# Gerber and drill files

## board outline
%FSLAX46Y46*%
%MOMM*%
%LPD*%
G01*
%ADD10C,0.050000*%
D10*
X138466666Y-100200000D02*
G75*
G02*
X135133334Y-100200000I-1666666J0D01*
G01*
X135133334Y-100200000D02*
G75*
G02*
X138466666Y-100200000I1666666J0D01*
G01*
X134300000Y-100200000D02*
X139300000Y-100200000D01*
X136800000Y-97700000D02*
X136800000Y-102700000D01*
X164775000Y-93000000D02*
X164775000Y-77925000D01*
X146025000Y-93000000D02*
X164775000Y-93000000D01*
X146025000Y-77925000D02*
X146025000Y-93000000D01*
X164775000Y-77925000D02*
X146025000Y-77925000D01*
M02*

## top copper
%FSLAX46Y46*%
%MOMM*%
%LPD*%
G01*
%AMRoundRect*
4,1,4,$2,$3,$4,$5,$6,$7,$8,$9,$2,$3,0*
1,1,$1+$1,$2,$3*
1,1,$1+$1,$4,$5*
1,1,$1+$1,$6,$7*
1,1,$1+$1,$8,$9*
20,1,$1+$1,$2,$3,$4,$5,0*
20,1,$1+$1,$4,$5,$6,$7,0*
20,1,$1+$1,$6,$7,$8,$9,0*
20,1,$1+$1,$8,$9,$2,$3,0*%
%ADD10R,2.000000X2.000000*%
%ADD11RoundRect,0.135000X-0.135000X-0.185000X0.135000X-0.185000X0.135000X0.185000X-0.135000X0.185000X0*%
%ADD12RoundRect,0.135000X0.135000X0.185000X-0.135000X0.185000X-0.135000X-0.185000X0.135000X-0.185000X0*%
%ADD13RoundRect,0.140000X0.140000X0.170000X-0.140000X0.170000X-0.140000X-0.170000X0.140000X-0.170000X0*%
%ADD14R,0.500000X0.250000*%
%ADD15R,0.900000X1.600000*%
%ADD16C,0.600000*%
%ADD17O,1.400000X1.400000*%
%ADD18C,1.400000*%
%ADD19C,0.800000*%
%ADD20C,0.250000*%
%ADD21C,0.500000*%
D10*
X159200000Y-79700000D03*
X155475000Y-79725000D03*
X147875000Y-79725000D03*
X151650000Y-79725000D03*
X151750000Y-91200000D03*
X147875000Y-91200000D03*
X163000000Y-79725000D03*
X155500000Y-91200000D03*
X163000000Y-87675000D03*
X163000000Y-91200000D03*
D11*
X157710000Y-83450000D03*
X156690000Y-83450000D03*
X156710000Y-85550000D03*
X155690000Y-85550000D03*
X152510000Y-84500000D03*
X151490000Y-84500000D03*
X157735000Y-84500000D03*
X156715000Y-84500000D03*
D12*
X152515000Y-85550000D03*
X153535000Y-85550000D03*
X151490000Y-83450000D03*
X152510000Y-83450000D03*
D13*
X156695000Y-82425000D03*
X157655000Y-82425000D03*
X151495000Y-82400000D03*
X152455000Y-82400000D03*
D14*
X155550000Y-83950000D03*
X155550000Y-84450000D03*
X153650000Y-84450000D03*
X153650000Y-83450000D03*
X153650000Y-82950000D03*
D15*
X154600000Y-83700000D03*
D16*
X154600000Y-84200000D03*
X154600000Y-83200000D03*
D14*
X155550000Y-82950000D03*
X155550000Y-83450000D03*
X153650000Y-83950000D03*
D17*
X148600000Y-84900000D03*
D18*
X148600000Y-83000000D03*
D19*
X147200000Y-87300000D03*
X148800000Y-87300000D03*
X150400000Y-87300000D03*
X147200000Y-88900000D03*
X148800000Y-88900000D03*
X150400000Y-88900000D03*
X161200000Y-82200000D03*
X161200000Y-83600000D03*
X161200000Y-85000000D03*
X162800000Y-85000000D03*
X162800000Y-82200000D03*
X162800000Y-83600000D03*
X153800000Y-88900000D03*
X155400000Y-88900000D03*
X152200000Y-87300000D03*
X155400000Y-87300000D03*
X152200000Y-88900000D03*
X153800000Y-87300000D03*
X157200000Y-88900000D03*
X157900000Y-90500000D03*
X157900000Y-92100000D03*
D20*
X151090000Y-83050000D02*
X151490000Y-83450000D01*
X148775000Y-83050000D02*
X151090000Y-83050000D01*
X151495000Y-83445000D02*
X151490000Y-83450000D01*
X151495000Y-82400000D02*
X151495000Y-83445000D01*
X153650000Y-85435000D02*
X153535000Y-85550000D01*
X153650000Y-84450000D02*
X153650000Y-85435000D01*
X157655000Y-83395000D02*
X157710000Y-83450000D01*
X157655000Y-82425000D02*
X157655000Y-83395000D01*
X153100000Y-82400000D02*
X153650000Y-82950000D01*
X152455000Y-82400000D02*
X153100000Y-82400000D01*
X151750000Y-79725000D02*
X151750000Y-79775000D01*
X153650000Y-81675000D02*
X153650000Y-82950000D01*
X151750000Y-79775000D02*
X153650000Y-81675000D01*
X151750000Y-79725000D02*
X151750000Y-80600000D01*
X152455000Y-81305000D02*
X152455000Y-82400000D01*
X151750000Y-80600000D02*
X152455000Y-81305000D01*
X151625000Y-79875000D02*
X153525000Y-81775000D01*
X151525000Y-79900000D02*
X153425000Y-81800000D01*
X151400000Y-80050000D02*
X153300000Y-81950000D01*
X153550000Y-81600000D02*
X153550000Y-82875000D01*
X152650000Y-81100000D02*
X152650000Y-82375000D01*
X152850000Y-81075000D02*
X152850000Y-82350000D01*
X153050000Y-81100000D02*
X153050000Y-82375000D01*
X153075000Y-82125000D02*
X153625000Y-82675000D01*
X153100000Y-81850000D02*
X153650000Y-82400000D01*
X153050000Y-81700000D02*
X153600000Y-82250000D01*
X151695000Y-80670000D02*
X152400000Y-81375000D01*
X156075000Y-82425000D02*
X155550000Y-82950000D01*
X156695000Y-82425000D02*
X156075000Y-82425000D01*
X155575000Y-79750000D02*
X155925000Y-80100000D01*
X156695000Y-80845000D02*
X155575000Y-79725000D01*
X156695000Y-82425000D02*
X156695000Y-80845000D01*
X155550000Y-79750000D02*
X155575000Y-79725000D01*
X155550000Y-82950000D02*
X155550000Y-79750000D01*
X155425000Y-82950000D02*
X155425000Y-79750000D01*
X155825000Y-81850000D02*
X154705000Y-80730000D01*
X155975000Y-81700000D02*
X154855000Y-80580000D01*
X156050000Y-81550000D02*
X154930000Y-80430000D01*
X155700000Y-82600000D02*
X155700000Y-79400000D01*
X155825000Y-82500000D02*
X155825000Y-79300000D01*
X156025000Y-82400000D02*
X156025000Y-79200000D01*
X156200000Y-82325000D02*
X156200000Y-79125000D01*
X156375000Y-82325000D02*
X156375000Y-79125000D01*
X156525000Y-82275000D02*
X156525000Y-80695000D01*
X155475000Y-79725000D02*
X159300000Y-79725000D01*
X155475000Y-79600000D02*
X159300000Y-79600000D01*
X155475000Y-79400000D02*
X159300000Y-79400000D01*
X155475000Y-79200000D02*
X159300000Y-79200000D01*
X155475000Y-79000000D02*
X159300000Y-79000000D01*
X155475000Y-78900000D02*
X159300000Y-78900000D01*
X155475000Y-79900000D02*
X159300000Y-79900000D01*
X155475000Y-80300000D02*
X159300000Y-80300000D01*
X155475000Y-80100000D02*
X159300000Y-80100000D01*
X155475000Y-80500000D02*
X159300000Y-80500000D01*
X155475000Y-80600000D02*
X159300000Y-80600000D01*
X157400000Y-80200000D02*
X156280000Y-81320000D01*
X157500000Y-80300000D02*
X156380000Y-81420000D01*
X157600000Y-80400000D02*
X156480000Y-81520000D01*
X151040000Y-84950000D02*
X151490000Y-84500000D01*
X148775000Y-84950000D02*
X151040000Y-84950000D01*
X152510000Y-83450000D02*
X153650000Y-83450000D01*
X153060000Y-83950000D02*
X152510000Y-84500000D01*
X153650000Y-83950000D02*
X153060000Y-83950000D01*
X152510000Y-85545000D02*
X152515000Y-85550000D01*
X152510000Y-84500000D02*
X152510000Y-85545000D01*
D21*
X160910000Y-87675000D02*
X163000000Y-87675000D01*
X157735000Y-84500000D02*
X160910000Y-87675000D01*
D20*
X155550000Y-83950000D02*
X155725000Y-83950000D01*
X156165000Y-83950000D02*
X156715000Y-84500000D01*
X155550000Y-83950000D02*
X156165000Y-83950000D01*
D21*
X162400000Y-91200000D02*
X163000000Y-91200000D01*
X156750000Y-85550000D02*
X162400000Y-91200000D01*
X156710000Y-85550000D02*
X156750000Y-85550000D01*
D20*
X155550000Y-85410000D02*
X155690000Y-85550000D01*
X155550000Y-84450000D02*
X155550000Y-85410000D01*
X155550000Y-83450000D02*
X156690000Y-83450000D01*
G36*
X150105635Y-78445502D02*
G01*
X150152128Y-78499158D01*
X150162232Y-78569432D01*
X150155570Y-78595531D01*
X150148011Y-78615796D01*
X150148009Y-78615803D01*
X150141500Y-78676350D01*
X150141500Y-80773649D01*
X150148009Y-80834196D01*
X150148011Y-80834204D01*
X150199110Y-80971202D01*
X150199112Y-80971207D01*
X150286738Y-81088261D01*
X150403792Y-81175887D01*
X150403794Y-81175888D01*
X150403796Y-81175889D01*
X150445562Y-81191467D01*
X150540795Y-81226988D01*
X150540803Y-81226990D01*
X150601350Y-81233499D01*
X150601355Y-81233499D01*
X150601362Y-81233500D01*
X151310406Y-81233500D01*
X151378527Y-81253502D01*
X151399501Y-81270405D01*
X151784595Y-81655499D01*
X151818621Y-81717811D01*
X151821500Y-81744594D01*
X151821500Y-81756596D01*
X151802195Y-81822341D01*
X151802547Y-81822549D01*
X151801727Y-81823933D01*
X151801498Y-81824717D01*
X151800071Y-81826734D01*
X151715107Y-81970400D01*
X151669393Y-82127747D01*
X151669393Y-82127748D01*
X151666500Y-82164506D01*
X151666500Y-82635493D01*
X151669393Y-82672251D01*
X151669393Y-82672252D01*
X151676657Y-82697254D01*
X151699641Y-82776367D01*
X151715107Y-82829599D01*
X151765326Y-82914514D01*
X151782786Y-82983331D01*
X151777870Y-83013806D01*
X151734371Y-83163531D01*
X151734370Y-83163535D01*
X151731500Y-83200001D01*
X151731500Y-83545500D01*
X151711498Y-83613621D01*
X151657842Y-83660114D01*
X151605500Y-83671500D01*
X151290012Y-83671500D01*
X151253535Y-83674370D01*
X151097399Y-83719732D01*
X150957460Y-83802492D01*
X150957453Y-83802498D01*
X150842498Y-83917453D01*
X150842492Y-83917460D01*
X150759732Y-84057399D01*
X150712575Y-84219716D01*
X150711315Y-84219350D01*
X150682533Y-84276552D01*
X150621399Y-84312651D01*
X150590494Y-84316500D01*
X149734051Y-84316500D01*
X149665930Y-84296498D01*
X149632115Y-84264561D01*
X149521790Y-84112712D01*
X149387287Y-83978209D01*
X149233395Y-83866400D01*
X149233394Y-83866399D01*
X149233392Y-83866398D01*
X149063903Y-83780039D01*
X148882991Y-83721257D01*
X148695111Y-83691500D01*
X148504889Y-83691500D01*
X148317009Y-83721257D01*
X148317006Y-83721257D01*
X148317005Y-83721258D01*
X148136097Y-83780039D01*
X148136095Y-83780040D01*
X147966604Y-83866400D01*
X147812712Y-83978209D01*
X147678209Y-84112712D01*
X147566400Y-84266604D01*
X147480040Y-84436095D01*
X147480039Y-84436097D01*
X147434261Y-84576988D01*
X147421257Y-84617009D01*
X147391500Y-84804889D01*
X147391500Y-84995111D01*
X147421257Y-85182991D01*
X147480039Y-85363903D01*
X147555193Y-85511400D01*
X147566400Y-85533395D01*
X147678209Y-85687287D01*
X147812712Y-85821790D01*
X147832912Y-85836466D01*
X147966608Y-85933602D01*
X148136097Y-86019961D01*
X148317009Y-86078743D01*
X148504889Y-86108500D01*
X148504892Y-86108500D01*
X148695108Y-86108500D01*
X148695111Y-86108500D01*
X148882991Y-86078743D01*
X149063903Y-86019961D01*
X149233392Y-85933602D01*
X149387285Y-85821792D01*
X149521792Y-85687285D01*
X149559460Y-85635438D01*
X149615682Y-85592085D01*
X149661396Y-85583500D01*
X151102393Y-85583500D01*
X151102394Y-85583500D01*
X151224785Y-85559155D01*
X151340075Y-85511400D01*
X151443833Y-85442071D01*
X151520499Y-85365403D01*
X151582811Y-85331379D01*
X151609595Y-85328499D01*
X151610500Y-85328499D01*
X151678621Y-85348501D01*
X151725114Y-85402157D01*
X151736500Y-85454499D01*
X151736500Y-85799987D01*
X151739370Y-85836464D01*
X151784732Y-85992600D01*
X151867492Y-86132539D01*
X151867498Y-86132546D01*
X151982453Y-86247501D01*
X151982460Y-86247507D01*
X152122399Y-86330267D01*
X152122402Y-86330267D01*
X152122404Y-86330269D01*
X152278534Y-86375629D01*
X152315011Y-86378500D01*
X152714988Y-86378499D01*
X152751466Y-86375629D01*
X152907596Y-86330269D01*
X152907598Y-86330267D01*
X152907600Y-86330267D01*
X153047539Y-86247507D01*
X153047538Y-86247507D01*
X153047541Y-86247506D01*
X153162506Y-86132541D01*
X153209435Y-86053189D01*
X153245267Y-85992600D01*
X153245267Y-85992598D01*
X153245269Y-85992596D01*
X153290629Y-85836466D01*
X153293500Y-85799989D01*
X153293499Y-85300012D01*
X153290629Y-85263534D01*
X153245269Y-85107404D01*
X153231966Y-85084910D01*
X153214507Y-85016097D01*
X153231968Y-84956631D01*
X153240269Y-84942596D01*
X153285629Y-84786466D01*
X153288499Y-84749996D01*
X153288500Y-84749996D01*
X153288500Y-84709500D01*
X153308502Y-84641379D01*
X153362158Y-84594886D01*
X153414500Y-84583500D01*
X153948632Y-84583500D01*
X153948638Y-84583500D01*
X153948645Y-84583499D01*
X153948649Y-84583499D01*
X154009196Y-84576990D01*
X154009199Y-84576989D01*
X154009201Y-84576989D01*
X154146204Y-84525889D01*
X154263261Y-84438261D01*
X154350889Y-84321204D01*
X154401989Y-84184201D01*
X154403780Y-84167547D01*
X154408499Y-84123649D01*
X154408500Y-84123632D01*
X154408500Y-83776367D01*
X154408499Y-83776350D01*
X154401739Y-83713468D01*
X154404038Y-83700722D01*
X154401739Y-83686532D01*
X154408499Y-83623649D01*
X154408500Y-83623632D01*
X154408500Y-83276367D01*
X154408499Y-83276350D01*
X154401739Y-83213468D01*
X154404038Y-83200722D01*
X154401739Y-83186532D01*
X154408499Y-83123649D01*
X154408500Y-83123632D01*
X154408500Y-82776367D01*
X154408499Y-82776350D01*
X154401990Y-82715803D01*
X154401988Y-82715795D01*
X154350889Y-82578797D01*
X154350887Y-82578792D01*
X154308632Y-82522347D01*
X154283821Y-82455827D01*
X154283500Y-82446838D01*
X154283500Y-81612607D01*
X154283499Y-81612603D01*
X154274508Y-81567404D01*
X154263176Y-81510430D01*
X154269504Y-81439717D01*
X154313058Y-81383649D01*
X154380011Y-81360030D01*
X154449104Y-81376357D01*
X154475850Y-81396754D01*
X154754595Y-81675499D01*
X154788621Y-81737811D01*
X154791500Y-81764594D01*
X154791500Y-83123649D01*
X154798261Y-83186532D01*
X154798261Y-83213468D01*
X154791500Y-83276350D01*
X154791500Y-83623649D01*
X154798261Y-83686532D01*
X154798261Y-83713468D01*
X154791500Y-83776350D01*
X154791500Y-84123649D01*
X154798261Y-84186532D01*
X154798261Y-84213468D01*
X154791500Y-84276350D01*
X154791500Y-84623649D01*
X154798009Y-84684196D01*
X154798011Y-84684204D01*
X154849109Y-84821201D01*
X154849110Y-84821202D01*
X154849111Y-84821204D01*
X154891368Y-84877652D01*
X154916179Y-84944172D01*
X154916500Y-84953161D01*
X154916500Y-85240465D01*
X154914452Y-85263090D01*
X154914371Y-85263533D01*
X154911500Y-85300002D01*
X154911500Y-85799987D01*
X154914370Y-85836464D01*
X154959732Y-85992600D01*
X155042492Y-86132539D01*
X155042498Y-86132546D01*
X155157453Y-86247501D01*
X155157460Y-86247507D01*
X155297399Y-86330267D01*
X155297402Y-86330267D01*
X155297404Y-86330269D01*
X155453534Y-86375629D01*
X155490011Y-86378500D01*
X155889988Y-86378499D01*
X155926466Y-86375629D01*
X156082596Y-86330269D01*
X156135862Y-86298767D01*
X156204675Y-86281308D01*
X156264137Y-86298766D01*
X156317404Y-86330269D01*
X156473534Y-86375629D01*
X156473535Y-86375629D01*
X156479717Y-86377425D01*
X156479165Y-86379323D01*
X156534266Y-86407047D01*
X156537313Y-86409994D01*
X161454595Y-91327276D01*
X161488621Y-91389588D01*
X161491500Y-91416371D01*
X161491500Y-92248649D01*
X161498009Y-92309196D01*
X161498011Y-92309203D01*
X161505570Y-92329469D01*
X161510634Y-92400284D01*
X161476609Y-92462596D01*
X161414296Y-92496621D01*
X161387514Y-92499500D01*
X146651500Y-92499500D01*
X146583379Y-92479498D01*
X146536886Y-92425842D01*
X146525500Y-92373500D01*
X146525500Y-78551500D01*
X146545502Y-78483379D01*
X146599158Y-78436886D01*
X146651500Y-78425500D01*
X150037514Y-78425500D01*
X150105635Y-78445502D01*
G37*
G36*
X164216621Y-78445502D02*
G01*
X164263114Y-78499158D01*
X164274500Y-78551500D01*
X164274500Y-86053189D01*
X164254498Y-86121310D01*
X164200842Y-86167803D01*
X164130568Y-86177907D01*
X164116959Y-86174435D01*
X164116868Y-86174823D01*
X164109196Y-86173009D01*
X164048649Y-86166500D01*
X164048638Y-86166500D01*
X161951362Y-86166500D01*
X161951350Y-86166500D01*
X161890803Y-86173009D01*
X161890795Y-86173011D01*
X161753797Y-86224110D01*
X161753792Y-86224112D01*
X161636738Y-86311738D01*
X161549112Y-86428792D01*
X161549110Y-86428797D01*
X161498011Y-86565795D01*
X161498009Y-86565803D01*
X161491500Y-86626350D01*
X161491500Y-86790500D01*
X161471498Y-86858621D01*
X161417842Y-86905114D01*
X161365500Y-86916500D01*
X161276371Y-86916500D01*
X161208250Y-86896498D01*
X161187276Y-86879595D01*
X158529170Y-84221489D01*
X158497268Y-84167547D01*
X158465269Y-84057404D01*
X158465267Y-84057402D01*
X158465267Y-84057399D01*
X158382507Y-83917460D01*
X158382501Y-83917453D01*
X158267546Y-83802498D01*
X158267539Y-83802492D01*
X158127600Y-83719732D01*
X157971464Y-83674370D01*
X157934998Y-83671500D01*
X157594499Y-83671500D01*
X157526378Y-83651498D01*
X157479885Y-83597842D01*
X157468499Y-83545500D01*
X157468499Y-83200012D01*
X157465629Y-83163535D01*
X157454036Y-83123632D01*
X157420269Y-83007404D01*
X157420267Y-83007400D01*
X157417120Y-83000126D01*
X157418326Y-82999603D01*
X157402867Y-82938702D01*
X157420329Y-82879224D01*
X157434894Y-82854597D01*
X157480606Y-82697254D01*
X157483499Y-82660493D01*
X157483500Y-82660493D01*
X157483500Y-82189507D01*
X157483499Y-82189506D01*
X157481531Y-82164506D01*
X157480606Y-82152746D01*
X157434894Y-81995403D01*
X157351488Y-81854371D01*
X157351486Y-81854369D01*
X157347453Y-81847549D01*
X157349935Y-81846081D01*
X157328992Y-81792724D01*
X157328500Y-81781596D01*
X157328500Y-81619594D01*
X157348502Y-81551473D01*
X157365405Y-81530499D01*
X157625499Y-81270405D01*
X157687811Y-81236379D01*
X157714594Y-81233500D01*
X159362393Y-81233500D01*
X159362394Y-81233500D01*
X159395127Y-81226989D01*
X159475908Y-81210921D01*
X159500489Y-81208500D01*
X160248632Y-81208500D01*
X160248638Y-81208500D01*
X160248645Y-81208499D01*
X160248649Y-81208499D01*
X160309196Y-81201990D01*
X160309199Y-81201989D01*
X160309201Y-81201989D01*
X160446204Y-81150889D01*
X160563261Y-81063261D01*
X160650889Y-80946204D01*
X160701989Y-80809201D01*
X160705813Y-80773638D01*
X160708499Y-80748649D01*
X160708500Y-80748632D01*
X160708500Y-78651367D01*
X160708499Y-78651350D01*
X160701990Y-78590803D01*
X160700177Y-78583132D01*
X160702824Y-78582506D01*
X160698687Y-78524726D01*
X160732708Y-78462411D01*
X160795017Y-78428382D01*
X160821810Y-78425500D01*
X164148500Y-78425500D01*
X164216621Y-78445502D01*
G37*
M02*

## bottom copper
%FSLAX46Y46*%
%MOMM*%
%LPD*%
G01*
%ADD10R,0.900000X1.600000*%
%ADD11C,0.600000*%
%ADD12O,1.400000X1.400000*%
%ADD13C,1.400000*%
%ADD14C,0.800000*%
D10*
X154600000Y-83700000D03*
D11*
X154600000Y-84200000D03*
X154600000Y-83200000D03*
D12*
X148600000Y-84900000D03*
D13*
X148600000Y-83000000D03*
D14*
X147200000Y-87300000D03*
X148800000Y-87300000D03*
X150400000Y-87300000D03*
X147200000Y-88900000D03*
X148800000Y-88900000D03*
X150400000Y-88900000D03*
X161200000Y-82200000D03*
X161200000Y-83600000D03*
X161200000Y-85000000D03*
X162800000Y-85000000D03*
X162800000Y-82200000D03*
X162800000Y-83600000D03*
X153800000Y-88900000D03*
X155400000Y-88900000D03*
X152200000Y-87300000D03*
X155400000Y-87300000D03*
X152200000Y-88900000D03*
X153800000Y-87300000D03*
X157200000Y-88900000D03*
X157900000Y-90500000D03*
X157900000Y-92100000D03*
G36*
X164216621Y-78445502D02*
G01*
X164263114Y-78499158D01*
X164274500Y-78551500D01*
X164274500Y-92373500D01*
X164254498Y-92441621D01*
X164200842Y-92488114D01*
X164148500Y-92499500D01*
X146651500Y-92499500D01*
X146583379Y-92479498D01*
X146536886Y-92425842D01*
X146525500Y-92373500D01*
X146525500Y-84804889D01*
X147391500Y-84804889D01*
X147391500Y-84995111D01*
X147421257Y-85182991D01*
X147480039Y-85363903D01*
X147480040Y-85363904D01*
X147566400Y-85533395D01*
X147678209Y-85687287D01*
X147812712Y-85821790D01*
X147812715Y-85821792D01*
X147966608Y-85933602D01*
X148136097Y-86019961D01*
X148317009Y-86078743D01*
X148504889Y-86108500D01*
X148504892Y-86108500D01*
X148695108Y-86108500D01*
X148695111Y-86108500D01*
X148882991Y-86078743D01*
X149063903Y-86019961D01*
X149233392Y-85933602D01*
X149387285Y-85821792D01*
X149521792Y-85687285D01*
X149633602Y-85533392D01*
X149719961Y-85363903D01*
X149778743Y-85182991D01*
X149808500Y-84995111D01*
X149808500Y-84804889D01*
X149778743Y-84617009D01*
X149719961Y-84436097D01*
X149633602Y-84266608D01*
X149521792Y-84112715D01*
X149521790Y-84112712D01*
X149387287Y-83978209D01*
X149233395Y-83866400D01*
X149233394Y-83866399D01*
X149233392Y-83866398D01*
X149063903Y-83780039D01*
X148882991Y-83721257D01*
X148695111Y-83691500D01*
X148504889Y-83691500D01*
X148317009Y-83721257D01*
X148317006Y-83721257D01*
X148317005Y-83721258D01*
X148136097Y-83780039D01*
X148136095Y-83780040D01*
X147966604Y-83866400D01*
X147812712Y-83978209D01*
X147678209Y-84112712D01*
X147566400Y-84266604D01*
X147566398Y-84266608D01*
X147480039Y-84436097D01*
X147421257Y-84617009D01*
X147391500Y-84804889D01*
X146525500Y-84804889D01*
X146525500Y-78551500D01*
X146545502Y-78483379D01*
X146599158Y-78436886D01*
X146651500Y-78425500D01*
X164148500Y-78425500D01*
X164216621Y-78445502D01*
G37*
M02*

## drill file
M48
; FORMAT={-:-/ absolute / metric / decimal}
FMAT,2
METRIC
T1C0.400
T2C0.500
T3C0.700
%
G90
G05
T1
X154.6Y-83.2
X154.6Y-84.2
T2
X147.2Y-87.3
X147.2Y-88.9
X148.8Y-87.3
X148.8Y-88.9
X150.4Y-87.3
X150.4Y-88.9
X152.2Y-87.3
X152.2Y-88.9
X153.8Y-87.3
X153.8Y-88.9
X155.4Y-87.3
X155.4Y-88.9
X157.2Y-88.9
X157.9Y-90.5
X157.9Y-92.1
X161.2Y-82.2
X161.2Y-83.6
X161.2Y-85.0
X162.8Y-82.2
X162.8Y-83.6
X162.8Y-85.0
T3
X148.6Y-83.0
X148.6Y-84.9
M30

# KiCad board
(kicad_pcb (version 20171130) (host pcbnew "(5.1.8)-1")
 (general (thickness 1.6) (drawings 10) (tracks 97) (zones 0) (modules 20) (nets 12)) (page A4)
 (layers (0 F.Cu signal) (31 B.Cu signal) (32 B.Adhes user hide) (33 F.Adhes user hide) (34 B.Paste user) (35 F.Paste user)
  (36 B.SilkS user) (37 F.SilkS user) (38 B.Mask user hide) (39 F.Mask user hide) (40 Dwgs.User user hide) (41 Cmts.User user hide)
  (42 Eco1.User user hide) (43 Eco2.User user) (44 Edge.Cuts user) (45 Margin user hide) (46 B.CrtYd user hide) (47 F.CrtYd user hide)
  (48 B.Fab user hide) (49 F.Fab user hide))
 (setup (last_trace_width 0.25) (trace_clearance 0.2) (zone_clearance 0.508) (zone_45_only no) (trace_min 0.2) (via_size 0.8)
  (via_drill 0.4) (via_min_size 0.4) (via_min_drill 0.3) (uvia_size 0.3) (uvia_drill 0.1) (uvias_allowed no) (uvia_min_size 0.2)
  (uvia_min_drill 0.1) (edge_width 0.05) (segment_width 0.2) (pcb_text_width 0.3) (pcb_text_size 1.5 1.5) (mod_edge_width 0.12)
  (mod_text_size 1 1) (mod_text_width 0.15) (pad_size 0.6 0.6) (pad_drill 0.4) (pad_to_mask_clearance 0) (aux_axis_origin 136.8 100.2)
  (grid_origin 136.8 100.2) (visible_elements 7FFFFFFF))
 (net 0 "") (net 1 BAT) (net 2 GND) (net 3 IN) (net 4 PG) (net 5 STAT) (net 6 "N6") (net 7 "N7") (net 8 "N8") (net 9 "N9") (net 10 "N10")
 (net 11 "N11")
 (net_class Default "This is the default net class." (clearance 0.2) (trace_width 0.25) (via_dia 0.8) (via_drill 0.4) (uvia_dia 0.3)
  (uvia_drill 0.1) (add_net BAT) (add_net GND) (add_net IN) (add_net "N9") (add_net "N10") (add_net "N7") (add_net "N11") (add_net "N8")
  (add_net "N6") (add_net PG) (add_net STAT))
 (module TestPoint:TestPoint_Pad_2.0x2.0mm (layer F.Cu) (at 159.2 79.7)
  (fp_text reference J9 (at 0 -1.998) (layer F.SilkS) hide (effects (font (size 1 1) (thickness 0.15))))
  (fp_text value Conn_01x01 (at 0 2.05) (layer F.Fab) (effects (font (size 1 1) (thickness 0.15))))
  (pad 1 smd rect (at 0 0) (size 2 2) (layers F.Cu F.Mask) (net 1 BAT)))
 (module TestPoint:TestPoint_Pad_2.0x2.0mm (layer F.Cu) (at 155.475 79.725)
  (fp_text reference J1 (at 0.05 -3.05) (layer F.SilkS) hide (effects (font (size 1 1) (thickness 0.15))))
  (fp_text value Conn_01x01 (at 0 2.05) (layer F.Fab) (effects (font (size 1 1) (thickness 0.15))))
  (pad 1 smd rect (at 0 0) (size 2 2) (layers F.Cu F.Mask) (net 1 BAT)))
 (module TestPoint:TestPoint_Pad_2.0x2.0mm (layer F.Cu) (at 147.875 79.725)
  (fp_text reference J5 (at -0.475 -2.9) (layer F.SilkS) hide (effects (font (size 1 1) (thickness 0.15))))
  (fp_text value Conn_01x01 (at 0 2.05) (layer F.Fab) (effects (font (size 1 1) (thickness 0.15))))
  (pad 1 smd rect (at 0 0) (size 2 2) (layers F.Cu F.Mask) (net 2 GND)))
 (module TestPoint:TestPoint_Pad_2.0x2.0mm (layer F.Cu) (at 151.65 79.725)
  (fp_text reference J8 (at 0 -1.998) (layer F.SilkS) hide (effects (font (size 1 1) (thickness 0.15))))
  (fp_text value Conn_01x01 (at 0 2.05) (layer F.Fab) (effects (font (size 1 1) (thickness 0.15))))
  (pad 1 smd rect (at 0 0) (size 2 2) (layers F.Cu F.Mask) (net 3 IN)))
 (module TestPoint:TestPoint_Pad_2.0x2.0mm (layer F.Cu) (at 151.75 91.2)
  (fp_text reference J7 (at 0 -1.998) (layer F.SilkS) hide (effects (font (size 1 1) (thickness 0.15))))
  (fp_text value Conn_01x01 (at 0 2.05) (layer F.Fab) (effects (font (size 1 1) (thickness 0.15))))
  (pad 1 smd rect (at 0 0) (size 2 2) (layers F.Cu F.Mask) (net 2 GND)))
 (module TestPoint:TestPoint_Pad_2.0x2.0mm (layer F.Cu) (at 147.875 91.2)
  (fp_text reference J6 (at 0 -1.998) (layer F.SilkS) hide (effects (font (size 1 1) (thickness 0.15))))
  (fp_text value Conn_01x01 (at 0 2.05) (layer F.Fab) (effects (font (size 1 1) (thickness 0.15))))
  (pad 1 smd rect (at 0 0) (size 2 2) (layers F.Cu F.Mask) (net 2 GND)))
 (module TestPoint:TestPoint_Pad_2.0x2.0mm (layer F.Cu) (at 163 79.725)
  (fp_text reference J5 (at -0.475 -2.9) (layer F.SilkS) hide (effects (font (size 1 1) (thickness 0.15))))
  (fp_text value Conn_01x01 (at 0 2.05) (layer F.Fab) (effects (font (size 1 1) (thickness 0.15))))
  (pad 1 smd rect (at 0 0) (size 2 2) (layers F.Cu F.Mask) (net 2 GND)))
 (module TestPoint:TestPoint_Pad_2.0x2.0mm (layer F.Cu) (at 155.5 91.2)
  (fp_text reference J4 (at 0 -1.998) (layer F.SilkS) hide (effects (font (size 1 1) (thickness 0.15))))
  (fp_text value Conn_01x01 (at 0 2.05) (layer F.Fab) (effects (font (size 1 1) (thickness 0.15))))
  (pad 1 smd rect (at 0 0) (size 2 2) (layers F.Cu F.Mask) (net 2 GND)))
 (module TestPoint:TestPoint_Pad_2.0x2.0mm (layer F.Cu) (at 163 87.675)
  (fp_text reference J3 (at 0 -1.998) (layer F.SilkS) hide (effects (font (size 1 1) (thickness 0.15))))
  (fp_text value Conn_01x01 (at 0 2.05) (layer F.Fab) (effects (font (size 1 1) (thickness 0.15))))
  (pad 1 smd rect (at 0 0) (size 2 2) (layers F.Cu F.Mask) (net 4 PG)))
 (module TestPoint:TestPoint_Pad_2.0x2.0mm (layer F.Cu) (at 163 91.2)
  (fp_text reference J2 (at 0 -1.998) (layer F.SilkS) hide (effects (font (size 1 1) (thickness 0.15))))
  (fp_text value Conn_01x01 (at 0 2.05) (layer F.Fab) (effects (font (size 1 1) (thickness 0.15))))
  (pad 1 smd rect (at 0 0) (size 2 2) (layers F.Cu F.Mask) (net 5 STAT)))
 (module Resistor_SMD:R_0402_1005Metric (layer F.Cu) (at 157.2 83.45)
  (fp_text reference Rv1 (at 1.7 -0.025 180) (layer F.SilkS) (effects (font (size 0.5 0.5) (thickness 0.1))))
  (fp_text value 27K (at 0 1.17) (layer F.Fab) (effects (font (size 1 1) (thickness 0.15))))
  (pad 2 smd roundrect (at 0.51 0) (size 0.54 0.64) (layers F.Cu F.Paste F.Mask) (roundrect_rratio 0.25) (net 2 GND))
  (pad 1 smd roundrect (at -0.51 0) (size 0.54 0.64) (layers F.Cu F.Paste F.Mask) (roundrect_rratio 0.25) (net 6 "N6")))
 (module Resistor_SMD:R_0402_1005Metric (layer F.Cu) (at 156.2 85.55)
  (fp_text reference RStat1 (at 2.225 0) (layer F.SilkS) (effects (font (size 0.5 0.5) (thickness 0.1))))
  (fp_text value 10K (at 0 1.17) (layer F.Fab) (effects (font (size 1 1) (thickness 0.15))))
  (pad 2 smd roundrect (at 0.51 0) (size 0.54 0.64) (layers F.Cu F.Paste F.Mask) (roundrect_rratio 0.25) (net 5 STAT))
  (pad 1 smd roundrect (at -0.51 0) (size 0.54 0.64) (layers F.Cu F.Paste F.Mask) (roundrect_rratio 0.25) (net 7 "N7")))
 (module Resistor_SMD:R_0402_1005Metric (layer F.Cu) (at 152 84.5)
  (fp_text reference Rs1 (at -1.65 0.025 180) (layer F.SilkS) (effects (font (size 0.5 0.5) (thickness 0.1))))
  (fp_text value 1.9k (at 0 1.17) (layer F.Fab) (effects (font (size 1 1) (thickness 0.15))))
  (pad 2 smd roundrect (at 0.51 0) (size 0.54 0.64) (layers F.Cu F.Paste F.Mask) (roundrect_rratio 0.25) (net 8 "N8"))
  (pad 1 smd roundrect (at -0.51 0) (size 0.54 0.64) (layers F.Cu F.Paste F.Mask) (roundrect_rratio 0.25) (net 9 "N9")))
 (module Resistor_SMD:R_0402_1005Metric (layer F.Cu) (at 157.225 84.5)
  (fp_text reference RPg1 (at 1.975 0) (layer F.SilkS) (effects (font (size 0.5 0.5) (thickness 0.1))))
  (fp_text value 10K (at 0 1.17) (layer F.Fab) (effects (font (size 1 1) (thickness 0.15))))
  (pad 2 smd roundrect (at 0.51 0) (size 0.54 0.64) (layers F.Cu F.Paste F.Mask) (roundrect_rratio 0.25) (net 4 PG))
  (pad 1 smd roundrect (at -0.51 0) (size 0.54 0.64) (layers F.Cu F.Paste F.Mask) (roundrect_rratio 0.25) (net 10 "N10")))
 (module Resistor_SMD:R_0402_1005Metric (layer F.Cu) (at 153.025 85.55 180)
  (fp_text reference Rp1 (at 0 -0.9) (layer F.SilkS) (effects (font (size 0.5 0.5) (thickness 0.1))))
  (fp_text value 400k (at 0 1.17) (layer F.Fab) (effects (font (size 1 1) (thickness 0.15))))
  (pad 2 smd roundrect (at 0.51 0 180) (size 0.54 0.64) (layers F.Cu F.Paste F.Mask) (roundrect_rratio 0.25) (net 8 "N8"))
  (pad 1 smd roundrect (at -0.51 0 180) (size 0.54 0.64) (layers F.Cu F.Paste F.Mask) (roundrect_rratio 0.25) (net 2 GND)))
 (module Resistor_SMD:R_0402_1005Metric (layer F.Cu) (at 152 83.45 180)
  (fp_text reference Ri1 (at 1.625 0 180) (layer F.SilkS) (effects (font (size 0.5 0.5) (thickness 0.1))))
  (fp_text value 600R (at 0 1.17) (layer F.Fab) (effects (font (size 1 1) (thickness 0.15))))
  (pad 2 smd roundrect (at 0.51 0 180) (size 0.54 0.64) (layers F.Cu F.Paste F.Mask) (roundrect_rratio 0.25) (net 2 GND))
  (pad 1 smd roundrect (at -0.51 0 180) (size 0.54 0.64) (layers F.Cu F.Paste F.Mask) (roundrect_rratio 0.25) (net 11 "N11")))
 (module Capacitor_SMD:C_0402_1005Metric (layer F.Cu) (at 157.175 82.425 180)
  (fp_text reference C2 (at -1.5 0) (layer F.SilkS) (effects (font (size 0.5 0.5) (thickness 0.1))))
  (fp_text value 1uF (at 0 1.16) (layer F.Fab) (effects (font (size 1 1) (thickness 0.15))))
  (pad 2 smd roundrect (at 0.48 0 180) (size 0.56 0.62) (layers F.Cu F.Paste F.Mask) (roundrect_rratio 0.25) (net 1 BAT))
  (pad 1 smd roundrect (at -0.48 0 180) (size 0.56 0.62) (layers F.Cu F.Paste F.Mask) (roundrect_rratio 0.25) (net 2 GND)))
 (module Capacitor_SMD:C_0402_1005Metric (layer F.Cu) (at 151.975 82.4 180)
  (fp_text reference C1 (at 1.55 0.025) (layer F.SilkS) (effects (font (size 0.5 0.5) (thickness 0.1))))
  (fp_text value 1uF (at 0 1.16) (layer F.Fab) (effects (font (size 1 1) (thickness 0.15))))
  (pad 2 smd roundrect (at 0.48 0 180) (size 0.56 0.62) (layers F.Cu F.Paste F.Mask) (roundrect_rratio 0.25) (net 2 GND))
  (pad 1 smd roundrect (at -0.48 0 180) (size 0.56 0.62) (layers F.Cu F.Paste F.Mask) (roundrect_rratio 0.25) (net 3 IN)))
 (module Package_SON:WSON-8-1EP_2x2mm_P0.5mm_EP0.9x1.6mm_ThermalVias (layer F.Cu) (at 154.6 83.7)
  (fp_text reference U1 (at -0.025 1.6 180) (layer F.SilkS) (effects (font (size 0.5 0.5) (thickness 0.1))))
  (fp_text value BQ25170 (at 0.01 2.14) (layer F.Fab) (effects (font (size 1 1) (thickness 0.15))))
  (pad "" smd rect (at 0 -0.4) (size 0.75 0.65) (layers F.Paste))
  (pad "" smd rect (at 0 0.4) (size 0.75 0.65) (layers F.Paste))
  (pad 9 smd rect (at 0 0) (size 0.9 1.6) (layers B.Cu) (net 2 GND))
  (pad 6 smd rect (at 0.95 0.25) (size 0.5 0.25) (layers F.Cu F.Paste F.Mask) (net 10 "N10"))
  (pad 5 smd rect (at 0.95 0.75) (size 0.5 0.25) (layers F.Cu F.Paste F.Mask) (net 7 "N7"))
  (pad 4 smd rect (at -0.95 0.75) (size 0.5 0.25) (layers F.Cu F.Paste F.Mask) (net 2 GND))
  (pad 2 smd rect (at -0.95 -0.25) (size 0.5 0.25) (layers F.Cu F.Paste F.Mask) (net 11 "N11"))
  (pad 1 smd rect (at -0.95 -0.75) (size 0.5 0.25) (layers F.Cu F.Paste F.Mask) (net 3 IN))
  (pad 9 smd rect (at 0 0) (size 0.9 1.6) (layers F.Cu F.Mask) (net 2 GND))
  (pad 9 thru_hole circle (at 0 0.5) (size 0.6 0.6) (drill 0.4) (layers *.Cu) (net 2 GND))
  (pad 9 thru_hole circle (at 0 -0.5) (size 0.6 0.6) (drill 0.4) (layers *.Cu) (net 2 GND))
  (pad 8 smd rect (at 0.95 -0.75) (size 0.5 0.25) (layers F.Cu F.Paste F.Mask) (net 1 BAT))
  (pad 7 smd rect (at 0.95 -0.25) (size 0.5 0.25) (layers F.Cu F.Paste F.Mask) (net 6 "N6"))
  (pad 3 smd rect (at -0.95 0.25) (size 0.5 0.25) (layers F.Cu F.Paste F.Mask) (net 8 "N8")))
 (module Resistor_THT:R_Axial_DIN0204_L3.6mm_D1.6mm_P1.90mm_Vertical (layer F.Cu) (at 148.6 83 270)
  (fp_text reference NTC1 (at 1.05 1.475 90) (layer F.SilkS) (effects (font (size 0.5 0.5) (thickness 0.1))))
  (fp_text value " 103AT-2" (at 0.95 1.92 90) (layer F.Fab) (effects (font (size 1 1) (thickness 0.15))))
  (pad 2 thru_hole oval (at 1.9 0 270) (size 1.4 1.4) (drill 0.7) (layers *.Cu *.Mask) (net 9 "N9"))
  (pad 1 thru_hole circle (at 0 0 270) (size 1.4 1.4) (drill 0.7) (layers *.Cu *.Mask) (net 2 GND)))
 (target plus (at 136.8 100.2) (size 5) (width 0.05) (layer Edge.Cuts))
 (gr_line (start 164.775 93) (end 164.775 77.925) (layer Edge.Cuts) (width 0.05))
 (gr_line (start 146.025 93) (end 164.775 93) (layer Edge.Cuts) (width 0.05))
 (gr_line (start 146.025 77.925) (end 146.025 93) (layer Edge.Cuts) (width 0.05))
 (gr_line (start 164.775 77.925) (end 146.025 77.925) (layer Edge.Cuts) (width 0.05))
 (segment (start 151.09 83.05) (end 151.49 83.45) (width 0.25) (layer F.Cu) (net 2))
 (segment (start 148.775 83.05) (end 151.09 83.05) (width 0.25) (layer F.Cu) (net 2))
 (segment (start 151.495 83.445) (end 151.49 83.45) (width 0.25) (layer F.Cu) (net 2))
 (segment (start 151.495 82.4) (end 151.495 83.445) (width 0.25) (layer F.Cu) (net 2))
 (segment (start 153.65 85.435) (end 153.535 85.55) (width 0.25) (layer F.Cu) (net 2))
 (segment (start 153.65 84.45) (end 153.65 85.435) (width 0.25) (layer F.Cu) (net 2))
 (segment (start 157.655 83.395) (end 157.71 83.45) (width 0.25) (layer F.Cu) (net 2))
 (segment (start 157.655 82.425) (end 157.655 83.395) (width 0.25) (layer F.Cu) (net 2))
 (via (at 147.2 87.3) (size 0.8) (drill 0.5) (layers F.Cu B.Cu) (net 2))
 (via (at 148.8 87.3) (size 0.8) (drill 0.5) (layers F.Cu B.Cu) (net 2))
 (via (at 150.4 87.3) (size 0.8) (drill 0.5) (layers F.Cu B.Cu) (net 2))
 (via (at 147.2 88.9) (size 0.8) (drill 0.5) (layers F.Cu B.Cu) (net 2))
 (via (at 148.8 88.9) (size 0.8) (drill 0.5) (layers F.Cu B.Cu) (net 2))
 (via (at 150.4 88.9) (size 0.8) (drill 0.5) (layers F.Cu B.Cu) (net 2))
 (via (at 161.2 82.2) (size 0.8) (drill 0.5) (layers F.Cu B.Cu) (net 2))
 (via (at 161.2 83.6) (size 0.8) (drill 0.5) (layers F.Cu B.Cu) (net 2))
 (via (at 161.2 85) (size 0.8) (drill 0.5) (layers F.Cu B.Cu) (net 2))
 (via (at 162.8 85) (size 0.8) (drill 0.5) (layers F.Cu B.Cu) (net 2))
 (via (at 162.8 82.2) (size 0.8) (drill 0.5) (layers F.Cu B.Cu) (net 2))
 (via (at 162.8 83.6) (size 0.8) (drill 0.5) (layers F.Cu B.Cu) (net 2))
 (via (at 153.8 88.9) (size 0.8) (drill 0.5) (layers F.Cu B.Cu) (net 2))
 (via (at 155.4 88.9) (size 0.8) (drill 0.5) (layers F.Cu B.Cu) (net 2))
 (via (at 152.2 87.3) (size 0.8) (drill 0.5) (layers F.Cu B.Cu) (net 2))
 (via (at 155.4 87.3) (size 0.8) (drill 0.5) (layers F.Cu B.Cu) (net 2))
 (via (at 152.2 88.9) (size 0.8) (drill 0.5) (layers F.Cu B.Cu) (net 2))
 (via (at 153.8 87.3) (size 0.8) (drill 0.5) (layers F.Cu B.Cu) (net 2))
 (via (at 157.2 88.9) (size 0.8) (drill 0.5) (layers F.Cu B.Cu) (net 2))
 (via (at 157.9 90.5) (size 0.8) (drill 0.5) (layers F.Cu B.Cu) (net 2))
 (via (at 157.9 92.1) (size 0.8) (drill 0.5) (layers F.Cu B.Cu) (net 2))
 (segment (start 153.1 82.4) (end 153.65 82.95) (width 0.25) (layer F.Cu) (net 3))
 (segment (start 152.455 82.4) (end 153.1 82.4) (width 0.25) (layer F.Cu) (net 3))
 (segment (start 151.75 79.725) (end 151.75 79.775) (width 0.25) (layer F.Cu) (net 3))
 (segment (start 153.65 81.675) (end 153.65 82.95) (width 0.25) (layer F.Cu) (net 3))
 (segment (start 151.75 79.775) (end 153.65 81.675) (width 0.25) (layer F.Cu) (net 3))
 (segment (start 151.75 79.725) (end 151.75 80.6) (width 0.25) (layer F.Cu) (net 3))
 (segment (start 152.455 81.305) (end 152.455 82.4) (width 0.25) (layer F.Cu) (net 3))
 (segment (start 151.75 80.6) (end 152.455 81.305) (width 0.25) (layer F.Cu) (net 3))
 (segment (start 151.625 79.875) (end 153.525 81.775) (width 0.25) (layer F.Cu) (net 3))
 (segment (start 151.525 79.9) (end 153.425 81.8) (width 0.25) (layer F.Cu) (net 3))
 (segment (start 151.4 80.05) (end 153.3 81.95) (width 0.25) (layer F.Cu) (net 3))
 (segment (start 153.55 81.6) (end 153.55 82.875) (width 0.25) (layer F.Cu) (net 3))
 (segment (start 152.65 81.1) (end 152.65 82.375) (width 0.25) (layer F.Cu) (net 3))
 (segment (start 152.85 81.075) (end 152.85 82.35) (width 0.25) (layer F.Cu) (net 3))
 (segment (start 153.05 81.1) (end 153.05 82.375) (width 0.25) (layer F.Cu) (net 3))
 (segment (start 153.075 82.125) (end 153.625 82.675) (width 0.25) (layer F.Cu) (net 3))
 (segment (start 153.1 81.85) (end 153.65 82.4) (width 0.25) (layer F.Cu) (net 3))
 (segment (start 153.05 81.7) (end 153.6 82.25) (width 0.25) (layer F.Cu) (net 3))
 (segment (start 151.695 80.67) (end 152.4 81.375) (width 0.25) (layer F.Cu) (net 3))
 (segment (start 156.075 82.425) (end 155.55 82.95) (width 0.25) (layer F.Cu) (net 1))
 (segment (start 156.695 82.425) (end 156.075 82.425) (width 0.25) (layer F.Cu) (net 1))
 (segment (start 155.575 79.75) (end 155.925 80.1) (width 0.25) (layer F.Cu) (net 1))
 (segment (start 156.695 80.845) (end 155.575 79.725) (width 0.25) (layer F.Cu) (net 1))
 (segment (start 156.695 82.425) (end 156.695 80.845) (width 0.25) (layer F.Cu) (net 1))
 (segment (start 155.55 79.75) (end 155.575 79.725) (width 0.25) (layer F.Cu) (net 1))
 (segment (start 155.55 82.95) (end 155.55 79.75) (width 0.25) (layer F.Cu) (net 1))
 (segment (start 155.425 82.95) (end 155.425 79.75) (width 0.25) (layer F.Cu) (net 1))
 (segment (start 155.825 81.85) (end 154.705 80.73) (width 0.25) (layer F.Cu) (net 1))
 (segment (start 155.975 81.7) (end 154.855 80.58) (width 0.25) (layer F.Cu) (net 1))
 (segment (start 156.05 81.55) (end 154.93 80.43) (width 0.25) (layer F.Cu) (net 1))
 (segment (start 155.7 82.6) (end 155.7 79.4) (width 0.25) (layer F.Cu) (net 1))
 (segment (start 155.825 82.5) (end 155.825 79.3) (width 0.25) (layer F.Cu) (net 1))
 (segment (start 156.025 82.4) (end 156.025 79.2) (width 0.25) (layer F.Cu) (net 1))
 (segment (start 156.2 82.325) (end 156.2 79.125) (width 0.25) (layer F.Cu) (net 1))
 (segment (start 156.375 82.325) (end 156.375 79.125) (width 0.25) (layer F.Cu) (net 1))
 (segment (start 156.525 82.275) (end 156.525 80.695) (width 0.25) (layer F.Cu) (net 1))
 (segment (start 155.475 79.725) (end 159.3 79.725) (width 0.25) (layer F.Cu) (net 1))
 (segment (start 155.475 79.6) (end 159.3 79.6) (width 0.25) (layer F.Cu) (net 1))
 (segment (start 155.475 79.4) (end 159.3 79.4) (width 0.25) (layer F.Cu) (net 1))
 (segment (start 155.475 79.2) (end 159.3 79.2) (width 0.25) (layer F.Cu) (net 1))
 (segment (start 155.475 79) (end 159.3 79) (width 0.25) (layer F.Cu) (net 1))
 (segment (start 155.475 78.9) (end 159.3 78.9) (width 0.25) (layer F.Cu) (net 1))
 (segment (start 155.475 79.9) (end 159.3 79.9) (width 0.25) (layer F.Cu) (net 1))
 (segment (start 155.475 80.3) (end 159.3 80.3) (width 0.25) (layer F.Cu) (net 1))
 (segment (start 155.475 80.1) (end 159.3 80.1) (width 0.25) (layer F.Cu) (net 1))
 (segment (start 155.475 80.5) (end 159.3 80.5) (width 0.25) (layer F.Cu) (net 1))
 (segment (start 155.475 80.6) (end 159.3 80.6) (width 0.25) (layer F.Cu) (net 1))
 (segment (start 157.4 80.2) (end 156.28 81.32) (width 0.25) (layer F.Cu) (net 1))
 (segment (start 157.5 80.3) (end 156.38 81.42) (width 0.25) (layer F.Cu) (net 1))
 (segment (start 157.6 80.4) (end 156.48 81.52) (width 0.25) (layer F.Cu) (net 1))
 (segment (start 151.04 84.95) (end 151.49 84.5) (width 0.25) (layer F.Cu) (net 9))
 (segment (start 148.775 84.95) (end 151.04 84.95) (width 0.25) (layer F.Cu) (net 9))
 (segment (start 152.51 83.45) (end 153.65 83.45) (width 0.25) (layer F.Cu) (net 11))
 (segment (start 153.06 83.95) (end 152.51 84.5) (width 0.25) (layer F.Cu) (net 8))
 (segment (start 153.65 83.95) (end 153.06 83.95) (width 0.25) (layer F.Cu) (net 8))
 (segment (start 152.51 85.545) (end 152.515 85.55) (width 0.25) (layer F.Cu) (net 8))
 (segment (start 152.51 84.5) (end 152.51 85.545) (width 0.25) (layer F.Cu) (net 8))
 (segment (start 160.91 87.675) (end 163 87.675) (width 0.5) (layer F.Cu) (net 4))
 (segment (start 157.735 84.5) (end 160.91 87.675) (width 0.5) (layer F.Cu) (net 4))
 (segment (start 155.55 83.95) (end 155.725 83.95) (width 0.25) (layer F.Cu) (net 10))
 (segment (start 156.165 83.95) (end 156.715 84.5) (width 0.25) (layer F.Cu) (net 10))
 (segment (start 155.55 83.95) (end 156.165 83.95) (width 0.25) (layer F.Cu) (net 10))
 (segment (start 162.4 91.2) (end 163 91.2) (width 0.5) (layer F.Cu) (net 5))
 (segment (start 156.75 85.55) (end 162.4 91.2) (width 0.5) (layer F.Cu) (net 5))
 (segment (start 156.71 85.55) (end 156.75 85.55) (width 0.5) (layer F.Cu) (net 5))
 (segment (start 155.55 85.41) (end 155.69 85.55) (width 0.25) (layer F.Cu) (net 7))
 (segment (start 155.55 84.45) (end 155.55 85.41) (width 0.25) (layer F.Cu) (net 7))
 (segment (start 155.55 83.45) (end 156.69 83.45) (width 0.25) (layer F.Cu) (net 6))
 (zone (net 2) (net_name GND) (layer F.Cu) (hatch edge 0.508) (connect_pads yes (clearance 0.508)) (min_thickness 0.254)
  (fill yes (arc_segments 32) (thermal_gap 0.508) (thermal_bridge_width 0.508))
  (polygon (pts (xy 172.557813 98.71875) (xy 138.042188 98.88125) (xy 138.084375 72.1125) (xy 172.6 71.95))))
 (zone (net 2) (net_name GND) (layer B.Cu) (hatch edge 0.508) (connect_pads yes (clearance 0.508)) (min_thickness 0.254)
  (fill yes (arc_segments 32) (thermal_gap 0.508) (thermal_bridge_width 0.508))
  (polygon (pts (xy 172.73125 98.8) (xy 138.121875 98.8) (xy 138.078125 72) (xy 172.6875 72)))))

